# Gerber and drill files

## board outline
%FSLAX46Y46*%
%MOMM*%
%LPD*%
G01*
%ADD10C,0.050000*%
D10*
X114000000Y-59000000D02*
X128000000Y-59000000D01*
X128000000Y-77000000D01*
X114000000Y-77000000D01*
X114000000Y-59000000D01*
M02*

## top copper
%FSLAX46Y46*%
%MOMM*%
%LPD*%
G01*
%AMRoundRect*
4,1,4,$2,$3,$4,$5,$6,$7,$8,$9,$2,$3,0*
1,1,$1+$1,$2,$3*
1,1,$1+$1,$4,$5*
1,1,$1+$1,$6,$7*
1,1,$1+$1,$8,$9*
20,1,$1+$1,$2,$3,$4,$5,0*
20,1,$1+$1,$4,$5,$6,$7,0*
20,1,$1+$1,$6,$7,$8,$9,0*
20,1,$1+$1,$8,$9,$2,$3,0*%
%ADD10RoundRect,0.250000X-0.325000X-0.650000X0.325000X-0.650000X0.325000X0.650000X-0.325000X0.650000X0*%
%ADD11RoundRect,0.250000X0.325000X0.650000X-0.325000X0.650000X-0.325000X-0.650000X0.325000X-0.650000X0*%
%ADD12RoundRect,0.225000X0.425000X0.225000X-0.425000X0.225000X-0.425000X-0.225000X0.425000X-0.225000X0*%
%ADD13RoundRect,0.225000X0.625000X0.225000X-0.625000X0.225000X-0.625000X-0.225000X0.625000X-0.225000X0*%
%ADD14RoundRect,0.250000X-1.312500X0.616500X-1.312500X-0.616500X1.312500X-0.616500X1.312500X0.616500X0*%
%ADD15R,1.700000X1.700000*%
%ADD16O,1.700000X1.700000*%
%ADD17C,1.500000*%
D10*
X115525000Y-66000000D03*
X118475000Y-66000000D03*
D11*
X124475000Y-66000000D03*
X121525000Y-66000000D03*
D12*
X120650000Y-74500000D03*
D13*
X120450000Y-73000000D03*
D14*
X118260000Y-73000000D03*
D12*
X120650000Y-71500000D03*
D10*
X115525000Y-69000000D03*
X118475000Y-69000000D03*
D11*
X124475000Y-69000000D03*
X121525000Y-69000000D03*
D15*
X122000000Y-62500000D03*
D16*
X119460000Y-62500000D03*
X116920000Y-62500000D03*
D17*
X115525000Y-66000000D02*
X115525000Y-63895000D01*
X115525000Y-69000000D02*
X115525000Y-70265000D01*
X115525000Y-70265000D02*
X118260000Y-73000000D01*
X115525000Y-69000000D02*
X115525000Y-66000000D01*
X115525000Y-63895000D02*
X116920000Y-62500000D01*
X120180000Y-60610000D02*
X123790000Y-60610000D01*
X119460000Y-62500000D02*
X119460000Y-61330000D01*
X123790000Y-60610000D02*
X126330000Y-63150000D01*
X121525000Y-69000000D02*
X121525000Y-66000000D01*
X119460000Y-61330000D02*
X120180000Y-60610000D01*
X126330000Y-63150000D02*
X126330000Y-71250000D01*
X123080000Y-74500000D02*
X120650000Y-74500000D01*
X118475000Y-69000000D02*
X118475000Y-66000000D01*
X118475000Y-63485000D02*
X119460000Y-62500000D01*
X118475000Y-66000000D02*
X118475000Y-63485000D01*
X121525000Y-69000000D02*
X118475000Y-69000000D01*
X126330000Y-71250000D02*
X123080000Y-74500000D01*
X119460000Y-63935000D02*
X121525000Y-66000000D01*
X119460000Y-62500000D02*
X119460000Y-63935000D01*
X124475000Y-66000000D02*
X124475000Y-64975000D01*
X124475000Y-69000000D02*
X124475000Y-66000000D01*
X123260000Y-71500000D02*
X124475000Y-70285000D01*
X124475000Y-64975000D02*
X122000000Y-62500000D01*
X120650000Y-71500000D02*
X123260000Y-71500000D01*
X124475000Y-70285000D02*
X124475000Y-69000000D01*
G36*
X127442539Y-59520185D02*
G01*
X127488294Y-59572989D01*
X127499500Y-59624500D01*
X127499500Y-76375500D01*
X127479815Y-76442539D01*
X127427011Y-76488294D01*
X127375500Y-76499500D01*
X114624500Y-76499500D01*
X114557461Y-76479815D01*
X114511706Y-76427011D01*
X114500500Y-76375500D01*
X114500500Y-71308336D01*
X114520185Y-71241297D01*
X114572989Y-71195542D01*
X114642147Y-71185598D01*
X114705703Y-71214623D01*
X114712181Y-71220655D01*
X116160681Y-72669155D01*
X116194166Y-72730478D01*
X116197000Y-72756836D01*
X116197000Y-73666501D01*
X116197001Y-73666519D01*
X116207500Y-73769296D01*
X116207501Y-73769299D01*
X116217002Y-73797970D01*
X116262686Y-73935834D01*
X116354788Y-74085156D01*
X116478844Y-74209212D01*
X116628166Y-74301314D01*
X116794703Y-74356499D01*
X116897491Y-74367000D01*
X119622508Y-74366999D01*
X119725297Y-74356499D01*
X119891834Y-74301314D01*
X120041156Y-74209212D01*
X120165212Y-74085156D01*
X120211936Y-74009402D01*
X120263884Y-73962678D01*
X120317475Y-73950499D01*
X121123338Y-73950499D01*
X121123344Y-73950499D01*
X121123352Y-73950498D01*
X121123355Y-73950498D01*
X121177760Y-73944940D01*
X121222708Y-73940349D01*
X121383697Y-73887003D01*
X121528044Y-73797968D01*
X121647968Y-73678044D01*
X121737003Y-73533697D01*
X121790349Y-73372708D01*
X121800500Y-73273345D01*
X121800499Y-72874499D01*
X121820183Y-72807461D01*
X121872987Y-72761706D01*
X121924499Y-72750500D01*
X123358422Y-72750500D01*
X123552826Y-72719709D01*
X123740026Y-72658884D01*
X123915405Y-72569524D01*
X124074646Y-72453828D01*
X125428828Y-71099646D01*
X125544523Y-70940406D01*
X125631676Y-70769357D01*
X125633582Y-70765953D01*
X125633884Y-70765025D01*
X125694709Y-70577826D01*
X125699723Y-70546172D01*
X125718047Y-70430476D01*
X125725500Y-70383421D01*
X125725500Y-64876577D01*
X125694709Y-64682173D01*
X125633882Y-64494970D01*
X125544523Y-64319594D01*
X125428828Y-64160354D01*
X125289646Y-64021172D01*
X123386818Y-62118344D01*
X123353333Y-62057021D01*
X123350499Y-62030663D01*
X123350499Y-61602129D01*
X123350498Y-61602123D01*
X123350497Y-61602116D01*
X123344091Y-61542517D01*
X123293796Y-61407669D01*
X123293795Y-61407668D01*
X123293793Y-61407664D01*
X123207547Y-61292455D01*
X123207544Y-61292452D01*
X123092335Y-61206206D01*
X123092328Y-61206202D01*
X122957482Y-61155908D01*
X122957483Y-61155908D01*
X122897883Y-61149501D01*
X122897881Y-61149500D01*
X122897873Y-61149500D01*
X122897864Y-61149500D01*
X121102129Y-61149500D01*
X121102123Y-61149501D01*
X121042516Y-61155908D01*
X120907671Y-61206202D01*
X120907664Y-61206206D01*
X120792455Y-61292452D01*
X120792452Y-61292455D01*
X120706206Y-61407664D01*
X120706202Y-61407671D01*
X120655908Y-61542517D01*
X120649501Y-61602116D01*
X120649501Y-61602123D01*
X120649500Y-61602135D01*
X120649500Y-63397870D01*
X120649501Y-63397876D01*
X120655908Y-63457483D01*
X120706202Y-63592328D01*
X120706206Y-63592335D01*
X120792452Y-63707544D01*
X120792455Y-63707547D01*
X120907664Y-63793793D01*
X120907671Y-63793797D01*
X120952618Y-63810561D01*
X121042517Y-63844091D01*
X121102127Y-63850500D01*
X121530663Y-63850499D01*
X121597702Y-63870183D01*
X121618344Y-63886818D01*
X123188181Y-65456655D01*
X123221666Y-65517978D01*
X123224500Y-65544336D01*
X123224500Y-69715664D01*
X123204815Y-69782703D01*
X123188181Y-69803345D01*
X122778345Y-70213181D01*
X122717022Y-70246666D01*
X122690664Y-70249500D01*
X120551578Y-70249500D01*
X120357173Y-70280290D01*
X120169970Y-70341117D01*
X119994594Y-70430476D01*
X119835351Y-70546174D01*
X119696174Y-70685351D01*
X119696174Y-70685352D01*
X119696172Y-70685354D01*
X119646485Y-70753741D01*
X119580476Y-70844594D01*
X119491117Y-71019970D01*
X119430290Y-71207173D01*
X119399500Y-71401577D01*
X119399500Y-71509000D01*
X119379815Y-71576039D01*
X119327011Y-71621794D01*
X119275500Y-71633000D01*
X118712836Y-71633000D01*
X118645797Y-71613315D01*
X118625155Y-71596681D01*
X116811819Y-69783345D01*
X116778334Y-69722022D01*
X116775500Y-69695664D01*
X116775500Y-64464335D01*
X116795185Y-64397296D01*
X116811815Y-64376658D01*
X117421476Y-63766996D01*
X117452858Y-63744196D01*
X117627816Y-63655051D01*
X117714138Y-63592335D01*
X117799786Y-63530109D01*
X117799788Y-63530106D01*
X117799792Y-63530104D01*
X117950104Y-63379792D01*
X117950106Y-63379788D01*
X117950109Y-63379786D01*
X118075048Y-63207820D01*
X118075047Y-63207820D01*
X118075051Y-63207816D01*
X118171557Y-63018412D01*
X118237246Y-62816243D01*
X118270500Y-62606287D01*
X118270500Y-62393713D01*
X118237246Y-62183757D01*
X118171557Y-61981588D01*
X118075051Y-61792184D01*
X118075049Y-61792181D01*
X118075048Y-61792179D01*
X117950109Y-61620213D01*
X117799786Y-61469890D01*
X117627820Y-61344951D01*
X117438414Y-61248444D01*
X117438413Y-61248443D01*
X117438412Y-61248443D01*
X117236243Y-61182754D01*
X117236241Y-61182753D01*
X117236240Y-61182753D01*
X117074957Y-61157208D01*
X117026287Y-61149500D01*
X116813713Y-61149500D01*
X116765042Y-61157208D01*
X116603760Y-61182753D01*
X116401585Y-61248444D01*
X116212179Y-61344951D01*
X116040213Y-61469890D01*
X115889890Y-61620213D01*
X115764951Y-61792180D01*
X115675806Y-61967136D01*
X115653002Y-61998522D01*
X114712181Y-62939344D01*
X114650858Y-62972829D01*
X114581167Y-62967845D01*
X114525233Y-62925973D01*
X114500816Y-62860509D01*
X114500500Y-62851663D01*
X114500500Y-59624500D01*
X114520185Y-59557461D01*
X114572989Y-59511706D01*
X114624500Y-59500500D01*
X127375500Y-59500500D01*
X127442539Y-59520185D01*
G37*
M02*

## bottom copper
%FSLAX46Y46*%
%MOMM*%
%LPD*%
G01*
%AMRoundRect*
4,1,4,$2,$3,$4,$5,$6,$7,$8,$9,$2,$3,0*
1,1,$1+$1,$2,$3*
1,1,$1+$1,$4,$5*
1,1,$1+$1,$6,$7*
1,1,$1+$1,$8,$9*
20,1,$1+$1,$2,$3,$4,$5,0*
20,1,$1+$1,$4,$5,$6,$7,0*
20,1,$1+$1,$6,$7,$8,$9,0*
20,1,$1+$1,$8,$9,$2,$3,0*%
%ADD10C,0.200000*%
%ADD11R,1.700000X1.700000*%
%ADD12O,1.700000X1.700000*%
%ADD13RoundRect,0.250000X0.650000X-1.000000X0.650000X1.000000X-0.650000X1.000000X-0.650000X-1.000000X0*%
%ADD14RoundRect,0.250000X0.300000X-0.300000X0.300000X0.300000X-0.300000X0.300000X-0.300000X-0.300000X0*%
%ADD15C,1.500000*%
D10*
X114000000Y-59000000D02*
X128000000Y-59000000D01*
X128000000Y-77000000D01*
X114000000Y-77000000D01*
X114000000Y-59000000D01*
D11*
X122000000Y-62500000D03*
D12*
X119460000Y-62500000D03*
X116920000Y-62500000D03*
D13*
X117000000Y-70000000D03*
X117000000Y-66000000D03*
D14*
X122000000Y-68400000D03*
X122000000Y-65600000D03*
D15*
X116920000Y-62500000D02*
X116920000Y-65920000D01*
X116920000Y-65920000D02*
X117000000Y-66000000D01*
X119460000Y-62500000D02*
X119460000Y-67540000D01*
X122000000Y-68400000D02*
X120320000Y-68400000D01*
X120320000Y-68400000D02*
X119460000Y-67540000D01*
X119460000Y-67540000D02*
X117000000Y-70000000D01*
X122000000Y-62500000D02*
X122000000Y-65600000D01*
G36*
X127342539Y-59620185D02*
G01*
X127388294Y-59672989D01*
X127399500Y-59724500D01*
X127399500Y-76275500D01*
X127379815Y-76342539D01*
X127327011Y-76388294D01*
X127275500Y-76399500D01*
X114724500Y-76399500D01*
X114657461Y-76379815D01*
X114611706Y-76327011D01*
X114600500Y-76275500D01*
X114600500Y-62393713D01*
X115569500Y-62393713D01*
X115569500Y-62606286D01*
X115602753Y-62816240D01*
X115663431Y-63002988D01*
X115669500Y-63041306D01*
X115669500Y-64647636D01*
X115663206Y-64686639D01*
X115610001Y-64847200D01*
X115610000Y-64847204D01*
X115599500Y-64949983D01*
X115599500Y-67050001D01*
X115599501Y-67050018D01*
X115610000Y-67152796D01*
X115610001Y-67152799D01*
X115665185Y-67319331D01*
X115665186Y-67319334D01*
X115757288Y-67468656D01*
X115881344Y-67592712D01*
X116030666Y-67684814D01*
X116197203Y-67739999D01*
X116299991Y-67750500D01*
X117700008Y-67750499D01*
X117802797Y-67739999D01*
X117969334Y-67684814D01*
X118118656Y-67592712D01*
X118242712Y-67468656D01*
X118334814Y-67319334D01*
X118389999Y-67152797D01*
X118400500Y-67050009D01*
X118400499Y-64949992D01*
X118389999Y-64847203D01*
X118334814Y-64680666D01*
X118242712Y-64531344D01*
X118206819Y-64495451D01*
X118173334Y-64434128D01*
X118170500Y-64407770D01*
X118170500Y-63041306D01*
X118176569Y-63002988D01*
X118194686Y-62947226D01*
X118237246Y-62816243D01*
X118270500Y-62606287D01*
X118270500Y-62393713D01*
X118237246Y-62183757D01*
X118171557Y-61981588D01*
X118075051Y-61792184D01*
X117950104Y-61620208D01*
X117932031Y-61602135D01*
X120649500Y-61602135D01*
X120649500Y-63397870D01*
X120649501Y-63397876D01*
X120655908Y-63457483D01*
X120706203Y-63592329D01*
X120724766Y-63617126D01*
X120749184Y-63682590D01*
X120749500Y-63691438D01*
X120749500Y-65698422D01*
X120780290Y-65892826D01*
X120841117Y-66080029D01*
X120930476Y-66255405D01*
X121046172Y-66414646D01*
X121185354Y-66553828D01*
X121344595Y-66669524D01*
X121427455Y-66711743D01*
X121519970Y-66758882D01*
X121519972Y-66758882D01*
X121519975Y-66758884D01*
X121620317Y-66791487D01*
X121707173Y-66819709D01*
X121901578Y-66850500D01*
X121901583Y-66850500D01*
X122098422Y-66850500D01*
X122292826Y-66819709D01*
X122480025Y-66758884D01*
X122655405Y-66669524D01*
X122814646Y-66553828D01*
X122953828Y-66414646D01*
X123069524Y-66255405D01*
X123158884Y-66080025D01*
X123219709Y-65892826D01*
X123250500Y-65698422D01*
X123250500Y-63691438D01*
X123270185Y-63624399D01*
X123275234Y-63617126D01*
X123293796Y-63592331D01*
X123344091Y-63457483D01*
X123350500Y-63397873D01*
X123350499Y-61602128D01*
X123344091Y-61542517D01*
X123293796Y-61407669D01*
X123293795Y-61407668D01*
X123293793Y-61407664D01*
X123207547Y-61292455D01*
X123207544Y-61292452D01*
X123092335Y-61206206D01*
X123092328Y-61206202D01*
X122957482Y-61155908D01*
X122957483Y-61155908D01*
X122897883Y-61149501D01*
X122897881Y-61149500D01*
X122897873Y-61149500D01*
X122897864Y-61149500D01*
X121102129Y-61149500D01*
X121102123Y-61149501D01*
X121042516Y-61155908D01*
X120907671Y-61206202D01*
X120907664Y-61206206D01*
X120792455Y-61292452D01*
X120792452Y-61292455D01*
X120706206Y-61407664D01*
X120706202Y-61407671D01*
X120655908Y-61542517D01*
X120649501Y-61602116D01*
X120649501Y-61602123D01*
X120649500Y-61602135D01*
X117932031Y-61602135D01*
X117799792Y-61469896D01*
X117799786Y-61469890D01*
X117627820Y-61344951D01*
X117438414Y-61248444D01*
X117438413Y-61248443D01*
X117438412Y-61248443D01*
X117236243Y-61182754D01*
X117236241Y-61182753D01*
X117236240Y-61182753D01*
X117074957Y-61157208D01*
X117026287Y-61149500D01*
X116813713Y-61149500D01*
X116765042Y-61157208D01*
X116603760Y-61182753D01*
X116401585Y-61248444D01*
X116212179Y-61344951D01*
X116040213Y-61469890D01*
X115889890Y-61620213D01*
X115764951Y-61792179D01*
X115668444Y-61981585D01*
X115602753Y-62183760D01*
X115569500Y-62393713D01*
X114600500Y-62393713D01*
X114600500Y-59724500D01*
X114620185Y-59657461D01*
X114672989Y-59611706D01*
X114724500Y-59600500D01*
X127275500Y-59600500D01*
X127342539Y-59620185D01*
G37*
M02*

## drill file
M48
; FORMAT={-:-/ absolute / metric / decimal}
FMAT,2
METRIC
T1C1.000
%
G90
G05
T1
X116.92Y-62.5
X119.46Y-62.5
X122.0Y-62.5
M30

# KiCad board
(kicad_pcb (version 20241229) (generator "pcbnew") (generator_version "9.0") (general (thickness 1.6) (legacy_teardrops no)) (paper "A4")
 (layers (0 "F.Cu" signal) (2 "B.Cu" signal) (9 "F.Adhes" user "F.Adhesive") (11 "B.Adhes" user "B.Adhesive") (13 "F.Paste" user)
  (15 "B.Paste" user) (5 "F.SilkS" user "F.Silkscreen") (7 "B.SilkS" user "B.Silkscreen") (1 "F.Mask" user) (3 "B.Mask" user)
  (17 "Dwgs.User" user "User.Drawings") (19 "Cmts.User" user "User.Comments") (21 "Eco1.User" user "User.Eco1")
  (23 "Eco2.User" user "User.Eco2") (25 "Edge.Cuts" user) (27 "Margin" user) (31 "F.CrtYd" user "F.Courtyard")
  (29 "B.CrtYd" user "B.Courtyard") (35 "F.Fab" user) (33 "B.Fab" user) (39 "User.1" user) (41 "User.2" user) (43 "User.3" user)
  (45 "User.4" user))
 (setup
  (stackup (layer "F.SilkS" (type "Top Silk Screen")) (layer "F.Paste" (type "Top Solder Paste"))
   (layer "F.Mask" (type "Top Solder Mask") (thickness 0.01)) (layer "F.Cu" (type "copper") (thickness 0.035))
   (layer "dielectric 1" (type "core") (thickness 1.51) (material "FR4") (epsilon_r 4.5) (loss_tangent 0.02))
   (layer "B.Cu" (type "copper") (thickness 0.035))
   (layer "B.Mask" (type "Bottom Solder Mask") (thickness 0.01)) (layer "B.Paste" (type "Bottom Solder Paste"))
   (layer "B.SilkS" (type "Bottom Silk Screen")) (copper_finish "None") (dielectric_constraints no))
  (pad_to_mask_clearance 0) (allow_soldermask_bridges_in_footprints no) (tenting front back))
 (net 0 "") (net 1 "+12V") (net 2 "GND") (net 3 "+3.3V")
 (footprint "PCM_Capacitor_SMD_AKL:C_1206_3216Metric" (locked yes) (layer "F.Cu") (at 117 66)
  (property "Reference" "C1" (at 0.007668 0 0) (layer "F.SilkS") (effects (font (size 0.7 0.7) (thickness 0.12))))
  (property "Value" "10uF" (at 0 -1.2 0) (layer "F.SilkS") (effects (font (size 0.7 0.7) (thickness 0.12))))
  (pad "1" smd roundrect (at -1.475 0) (size 1.15 1.8) (layers "F.Cu" "F.Mask" "F.Paste") (roundrect_rratio 0.217391) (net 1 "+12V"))
  (pad "2" smd roundrect (at 1.475 0) (size 1.15 1.8) (layers "F.Cu" "F.Mask" "F.Paste") (roundrect_rratio 0.217391) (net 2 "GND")))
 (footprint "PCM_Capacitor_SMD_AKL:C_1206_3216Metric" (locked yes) (layer "F.Cu") (at 123 66 180)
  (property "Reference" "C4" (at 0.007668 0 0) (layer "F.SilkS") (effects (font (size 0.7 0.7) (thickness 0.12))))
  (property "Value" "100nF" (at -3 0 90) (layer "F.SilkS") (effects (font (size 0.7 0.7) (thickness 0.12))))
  (pad "1" smd roundrect (at -1.475 0 180) (size 1.15 1.8) (layers "F.Cu" "F.Mask" "F.Paste") (roundrect_rratio 0.217391) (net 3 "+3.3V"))
  (pad "2" smd roundrect (at 1.475 0 180) (size 1.15 1.8) (layers "F.Cu" "F.Mask" "F.Paste") (roundrect_rratio 0.217391) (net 2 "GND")))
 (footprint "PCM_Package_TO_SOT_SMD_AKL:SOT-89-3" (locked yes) (layer "F.Cu") (at 119 73 180)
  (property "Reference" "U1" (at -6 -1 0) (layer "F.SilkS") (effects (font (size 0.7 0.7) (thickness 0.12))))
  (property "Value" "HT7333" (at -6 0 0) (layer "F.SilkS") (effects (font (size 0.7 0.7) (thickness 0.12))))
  (pad "1" smd roundrect (at -1.65 -1.5 180) (size 1.3 0.9) (layers "F.Cu" "F.Mask" "F.Paste") (roundrect_rratio 0.25) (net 2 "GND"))
  (pad "2" smd roundrect (at -1.45 0 180) (size 1.7 0.9) (layers "F.Cu" "F.Mask" "F.Paste") (roundrect_rratio 0.25) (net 1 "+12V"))
  (pad "2" smd roundrect (at 0.74 0 270) (size 1.733 3.125) (layers "F.Cu" "F.Mask" "F.Paste") (roundrect_rratio 0.1442585113)
   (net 1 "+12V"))
  (pad "3" smd roundrect (at -1.65 1.5 180) (size 1.3 0.9) (layers "F.Cu" "F.Mask" "F.Paste") (roundrect_rratio 0.25) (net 3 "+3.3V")))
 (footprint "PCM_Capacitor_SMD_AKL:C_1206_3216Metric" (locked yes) (layer "F.Cu") (at 117 69)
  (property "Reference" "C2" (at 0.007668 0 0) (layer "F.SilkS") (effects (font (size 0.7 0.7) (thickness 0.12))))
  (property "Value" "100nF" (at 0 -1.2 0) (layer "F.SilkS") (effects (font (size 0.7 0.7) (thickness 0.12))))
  (pad "1" smd roundrect (at -1.475 0) (size 1.15 1.8) (layers "F.Cu" "F.Mask" "F.Paste") (roundrect_rratio 0.217391) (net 1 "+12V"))
  (pad "2" smd roundrect (at 1.475 0) (size 1.15 1.8) (layers "F.Cu" "F.Mask" "F.Paste") (roundrect_rratio 0.217391) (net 2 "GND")))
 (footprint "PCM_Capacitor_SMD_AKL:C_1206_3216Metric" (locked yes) (layer "F.Cu") (at 123 69 180)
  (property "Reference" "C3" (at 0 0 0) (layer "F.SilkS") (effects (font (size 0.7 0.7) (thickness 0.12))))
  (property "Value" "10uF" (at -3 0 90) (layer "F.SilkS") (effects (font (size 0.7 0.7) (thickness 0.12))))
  (pad "1" smd roundrect (at -1.475 0 180) (size 1.15 1.8) (layers "F.Cu" "F.Mask" "F.Paste") (roundrect_rratio 0.217391) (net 3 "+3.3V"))
  (pad "2" smd roundrect (at 1.475 0 180) (size 1.15 1.8) (layers "F.Cu" "F.Mask" "F.Paste") (roundrect_rratio 0.217391) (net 2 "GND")))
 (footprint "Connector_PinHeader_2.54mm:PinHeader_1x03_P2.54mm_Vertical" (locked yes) (layer "F.Cu") (at 122 62.5 -90)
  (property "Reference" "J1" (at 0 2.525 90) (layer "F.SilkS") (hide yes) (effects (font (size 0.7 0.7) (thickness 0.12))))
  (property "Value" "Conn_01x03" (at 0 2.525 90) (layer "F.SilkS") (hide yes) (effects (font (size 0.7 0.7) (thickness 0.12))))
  (pad "1" thru_hole rect (at 0 0 270) (size 1.7 1.7) (drill 1) (layers "*.Cu" "*.Mask") (remove_unused_layers no) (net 3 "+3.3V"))
  (pad "2" thru_hole oval (at 0 2.54 270) (size 1.7 1.7) (drill 1) (layers "*.Cu" "*.Mask") (remove_unused_layers no) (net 2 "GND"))
  (pad "3" thru_hole oval (at 0 5.08 270) (size 1.7 1.7) (drill 1) (layers "*.Cu" "*.Mask") (remove_unused_layers no) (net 1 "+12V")))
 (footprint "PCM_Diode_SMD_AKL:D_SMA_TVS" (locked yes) (layer "B.Cu") (at 117 68 90)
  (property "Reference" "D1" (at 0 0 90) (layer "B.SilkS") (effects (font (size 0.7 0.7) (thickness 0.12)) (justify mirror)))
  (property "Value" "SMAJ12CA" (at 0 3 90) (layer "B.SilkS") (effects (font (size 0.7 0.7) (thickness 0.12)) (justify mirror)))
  (pad "1" smd roundrect (at -2 0 90) (size 2.5 1.8) (layers "B.Cu" "B.Mask" "B.Paste") (roundrect_rratio 0.1388888889) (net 2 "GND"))
  (pad "2" smd roundrect (at 2 0 90) (size 2.5 1.8) (layers "B.Cu" "B.Mask" "B.Paste") (roundrect_rratio 0.1388888889) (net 1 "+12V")))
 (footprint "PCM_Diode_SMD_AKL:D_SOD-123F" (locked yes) (layer "B.Cu") (at 122 67 90)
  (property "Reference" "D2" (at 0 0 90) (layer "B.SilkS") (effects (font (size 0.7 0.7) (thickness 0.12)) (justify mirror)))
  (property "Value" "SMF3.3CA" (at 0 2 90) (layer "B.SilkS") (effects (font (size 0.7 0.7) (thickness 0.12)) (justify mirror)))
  (pad "1" smd roundrect (at -1.4 0 90) (size 1.1 1.1) (layers "B.Cu" "B.Mask" "B.Paste") (roundrect_rratio 0.2272727273) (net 2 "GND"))
  (pad "2" smd roundrect (at 1.4 0 90) (size 1.1 1.1) (layers "B.Cu" "B.Mask" "B.Paste") (roundrect_rratio 0.2272727273) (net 3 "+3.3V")))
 (gr_rect (start 114 59) (end 128 77) (stroke (width 0.2) (type default)) (fill no) (locked yes) (layer "B.Cu"))
 (gr_rect (start 114 59) (end 128 77) (stroke (width 0.05) (type default)) (fill no) (locked yes) (layer "Edge.Cuts"))
 (segment (start 115.525 66) (end 115.525 63.895) (width 1.5) (locked yes) (layer "F.Cu") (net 1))
 (segment (start 115.525 69) (end 115.525 70.265) (width 1.5) (locked yes) (layer "F.Cu") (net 1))
 (segment (start 115.525 70.265) (end 118.26 73) (width 1.5) (locked yes) (layer "F.Cu") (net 1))
 (segment (start 115.525 69) (end 115.525 66) (width 1.5) (locked yes) (layer "F.Cu") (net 1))
 (segment (start 115.525 63.895) (end 116.92 62.5) (width 1.5) (locked yes) (layer "F.Cu") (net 1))
 (segment (start 116.92 62.5) (end 116.92 65.92) (width 1.5) (locked yes) (layer "B.Cu") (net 1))
 (segment (start 116.92 65.92) (end 117 66) (width 1.5) (locked yes) (layer "B.Cu") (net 1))
 (segment (start 120.18 60.61) (end 123.79 60.61) (width 1.5) (locked yes) (layer "F.Cu") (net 2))
 (segment (start 119.46 62.5) (end 119.46 61.33) (width 1.5) (locked yes) (layer "F.Cu") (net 2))
 (segment (start 123.79 60.61) (end 126.33 63.15) (width 1.5) (locked yes) (layer "F.Cu") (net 2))
 (segment (start 121.525 69) (end 121.525 66) (width 1.5) (locked yes) (layer "F.Cu") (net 2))
 (segment (start 119.46 61.33) (end 120.18 60.61) (width 1.5) (locked yes) (layer "F.Cu") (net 2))
 (segment (start 126.33 63.15) (end 126.33 71.25) (width 1.5) (locked yes) (layer "F.Cu") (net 2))
 (segment (start 123.08 74.5) (end 120.65 74.5) (width 1.5) (locked yes) (layer "F.Cu") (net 2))
 (segment (start 118.475 69) (end 118.475 66) (width 1.5) (locked yes) (layer "F.Cu") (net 2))
 (segment (start 118.475 63.485) (end 119.46 62.5) (width 1.5) (locked yes) (layer "F.Cu") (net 2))
 (segment (start 118.475 66) (end 118.475 63.485) (width 1.5) (locked yes) (layer "F.Cu") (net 2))
 (segment (start 121.525 69) (end 118.475 69) (width 1.5) (locked yes) (layer "F.Cu") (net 2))
 (segment (start 126.33 71.25) (end 123.08 74.5) (width 1.5) (locked yes) (layer "F.Cu") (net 2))
 (segment (start 119.46 63.935) (end 121.525 66) (width 1.5) (locked yes) (layer "F.Cu") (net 2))
 (segment (start 119.46 62.5) (end 119.46 63.935) (width 1.5) (locked yes) (layer "F.Cu") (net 2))
 (segment (start 119.46 62.5) (end 119.46 67.54) (width 1.5) (locked yes) (layer "B.Cu") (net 2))
 (segment (start 122 68.4) (end 120.32 68.4) (width 1.5) (locked yes) (layer "B.Cu") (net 2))
 (segment (start 120.32 68.4) (end 119.46 67.54) (width 1.5) (locked yes) (layer "B.Cu") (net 2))
 (segment (start 119.46 67.54) (end 117 70) (width 1.5) (locked yes) (layer "B.Cu") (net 2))
 (segment (start 124.475 66) (end 124.475 64.975) (width 1.5) (locked yes) (layer "F.Cu") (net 3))
 (segment (start 124.475 69) (end 124.475 66) (width 1.5) (locked yes) (layer "F.Cu") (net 3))
 (segment (start 123.26 71.5) (end 124.475 70.285) (width 1.5) (locked yes) (layer "F.Cu") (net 3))
 (segment (start 124.475 64.975) (end 122 62.5) (width 1.5) (locked yes) (layer "F.Cu") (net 3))
 (segment (start 120.65 71.5) (end 123.26 71.5) (width 1.5) (locked yes) (layer "F.Cu") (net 3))
 (segment (start 124.475 70.285) (end 124.475 69) (width 1.5) (locked yes) (layer "F.Cu") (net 3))
 (segment (start 122 62.5) (end 122 65.6) (width 1.5) (locked yes) (layer "B.Cu") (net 3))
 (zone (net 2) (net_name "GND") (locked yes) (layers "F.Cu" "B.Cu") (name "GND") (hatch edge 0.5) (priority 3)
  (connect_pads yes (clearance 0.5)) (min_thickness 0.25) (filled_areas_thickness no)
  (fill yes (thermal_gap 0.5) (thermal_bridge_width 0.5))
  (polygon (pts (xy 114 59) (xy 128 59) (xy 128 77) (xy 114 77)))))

